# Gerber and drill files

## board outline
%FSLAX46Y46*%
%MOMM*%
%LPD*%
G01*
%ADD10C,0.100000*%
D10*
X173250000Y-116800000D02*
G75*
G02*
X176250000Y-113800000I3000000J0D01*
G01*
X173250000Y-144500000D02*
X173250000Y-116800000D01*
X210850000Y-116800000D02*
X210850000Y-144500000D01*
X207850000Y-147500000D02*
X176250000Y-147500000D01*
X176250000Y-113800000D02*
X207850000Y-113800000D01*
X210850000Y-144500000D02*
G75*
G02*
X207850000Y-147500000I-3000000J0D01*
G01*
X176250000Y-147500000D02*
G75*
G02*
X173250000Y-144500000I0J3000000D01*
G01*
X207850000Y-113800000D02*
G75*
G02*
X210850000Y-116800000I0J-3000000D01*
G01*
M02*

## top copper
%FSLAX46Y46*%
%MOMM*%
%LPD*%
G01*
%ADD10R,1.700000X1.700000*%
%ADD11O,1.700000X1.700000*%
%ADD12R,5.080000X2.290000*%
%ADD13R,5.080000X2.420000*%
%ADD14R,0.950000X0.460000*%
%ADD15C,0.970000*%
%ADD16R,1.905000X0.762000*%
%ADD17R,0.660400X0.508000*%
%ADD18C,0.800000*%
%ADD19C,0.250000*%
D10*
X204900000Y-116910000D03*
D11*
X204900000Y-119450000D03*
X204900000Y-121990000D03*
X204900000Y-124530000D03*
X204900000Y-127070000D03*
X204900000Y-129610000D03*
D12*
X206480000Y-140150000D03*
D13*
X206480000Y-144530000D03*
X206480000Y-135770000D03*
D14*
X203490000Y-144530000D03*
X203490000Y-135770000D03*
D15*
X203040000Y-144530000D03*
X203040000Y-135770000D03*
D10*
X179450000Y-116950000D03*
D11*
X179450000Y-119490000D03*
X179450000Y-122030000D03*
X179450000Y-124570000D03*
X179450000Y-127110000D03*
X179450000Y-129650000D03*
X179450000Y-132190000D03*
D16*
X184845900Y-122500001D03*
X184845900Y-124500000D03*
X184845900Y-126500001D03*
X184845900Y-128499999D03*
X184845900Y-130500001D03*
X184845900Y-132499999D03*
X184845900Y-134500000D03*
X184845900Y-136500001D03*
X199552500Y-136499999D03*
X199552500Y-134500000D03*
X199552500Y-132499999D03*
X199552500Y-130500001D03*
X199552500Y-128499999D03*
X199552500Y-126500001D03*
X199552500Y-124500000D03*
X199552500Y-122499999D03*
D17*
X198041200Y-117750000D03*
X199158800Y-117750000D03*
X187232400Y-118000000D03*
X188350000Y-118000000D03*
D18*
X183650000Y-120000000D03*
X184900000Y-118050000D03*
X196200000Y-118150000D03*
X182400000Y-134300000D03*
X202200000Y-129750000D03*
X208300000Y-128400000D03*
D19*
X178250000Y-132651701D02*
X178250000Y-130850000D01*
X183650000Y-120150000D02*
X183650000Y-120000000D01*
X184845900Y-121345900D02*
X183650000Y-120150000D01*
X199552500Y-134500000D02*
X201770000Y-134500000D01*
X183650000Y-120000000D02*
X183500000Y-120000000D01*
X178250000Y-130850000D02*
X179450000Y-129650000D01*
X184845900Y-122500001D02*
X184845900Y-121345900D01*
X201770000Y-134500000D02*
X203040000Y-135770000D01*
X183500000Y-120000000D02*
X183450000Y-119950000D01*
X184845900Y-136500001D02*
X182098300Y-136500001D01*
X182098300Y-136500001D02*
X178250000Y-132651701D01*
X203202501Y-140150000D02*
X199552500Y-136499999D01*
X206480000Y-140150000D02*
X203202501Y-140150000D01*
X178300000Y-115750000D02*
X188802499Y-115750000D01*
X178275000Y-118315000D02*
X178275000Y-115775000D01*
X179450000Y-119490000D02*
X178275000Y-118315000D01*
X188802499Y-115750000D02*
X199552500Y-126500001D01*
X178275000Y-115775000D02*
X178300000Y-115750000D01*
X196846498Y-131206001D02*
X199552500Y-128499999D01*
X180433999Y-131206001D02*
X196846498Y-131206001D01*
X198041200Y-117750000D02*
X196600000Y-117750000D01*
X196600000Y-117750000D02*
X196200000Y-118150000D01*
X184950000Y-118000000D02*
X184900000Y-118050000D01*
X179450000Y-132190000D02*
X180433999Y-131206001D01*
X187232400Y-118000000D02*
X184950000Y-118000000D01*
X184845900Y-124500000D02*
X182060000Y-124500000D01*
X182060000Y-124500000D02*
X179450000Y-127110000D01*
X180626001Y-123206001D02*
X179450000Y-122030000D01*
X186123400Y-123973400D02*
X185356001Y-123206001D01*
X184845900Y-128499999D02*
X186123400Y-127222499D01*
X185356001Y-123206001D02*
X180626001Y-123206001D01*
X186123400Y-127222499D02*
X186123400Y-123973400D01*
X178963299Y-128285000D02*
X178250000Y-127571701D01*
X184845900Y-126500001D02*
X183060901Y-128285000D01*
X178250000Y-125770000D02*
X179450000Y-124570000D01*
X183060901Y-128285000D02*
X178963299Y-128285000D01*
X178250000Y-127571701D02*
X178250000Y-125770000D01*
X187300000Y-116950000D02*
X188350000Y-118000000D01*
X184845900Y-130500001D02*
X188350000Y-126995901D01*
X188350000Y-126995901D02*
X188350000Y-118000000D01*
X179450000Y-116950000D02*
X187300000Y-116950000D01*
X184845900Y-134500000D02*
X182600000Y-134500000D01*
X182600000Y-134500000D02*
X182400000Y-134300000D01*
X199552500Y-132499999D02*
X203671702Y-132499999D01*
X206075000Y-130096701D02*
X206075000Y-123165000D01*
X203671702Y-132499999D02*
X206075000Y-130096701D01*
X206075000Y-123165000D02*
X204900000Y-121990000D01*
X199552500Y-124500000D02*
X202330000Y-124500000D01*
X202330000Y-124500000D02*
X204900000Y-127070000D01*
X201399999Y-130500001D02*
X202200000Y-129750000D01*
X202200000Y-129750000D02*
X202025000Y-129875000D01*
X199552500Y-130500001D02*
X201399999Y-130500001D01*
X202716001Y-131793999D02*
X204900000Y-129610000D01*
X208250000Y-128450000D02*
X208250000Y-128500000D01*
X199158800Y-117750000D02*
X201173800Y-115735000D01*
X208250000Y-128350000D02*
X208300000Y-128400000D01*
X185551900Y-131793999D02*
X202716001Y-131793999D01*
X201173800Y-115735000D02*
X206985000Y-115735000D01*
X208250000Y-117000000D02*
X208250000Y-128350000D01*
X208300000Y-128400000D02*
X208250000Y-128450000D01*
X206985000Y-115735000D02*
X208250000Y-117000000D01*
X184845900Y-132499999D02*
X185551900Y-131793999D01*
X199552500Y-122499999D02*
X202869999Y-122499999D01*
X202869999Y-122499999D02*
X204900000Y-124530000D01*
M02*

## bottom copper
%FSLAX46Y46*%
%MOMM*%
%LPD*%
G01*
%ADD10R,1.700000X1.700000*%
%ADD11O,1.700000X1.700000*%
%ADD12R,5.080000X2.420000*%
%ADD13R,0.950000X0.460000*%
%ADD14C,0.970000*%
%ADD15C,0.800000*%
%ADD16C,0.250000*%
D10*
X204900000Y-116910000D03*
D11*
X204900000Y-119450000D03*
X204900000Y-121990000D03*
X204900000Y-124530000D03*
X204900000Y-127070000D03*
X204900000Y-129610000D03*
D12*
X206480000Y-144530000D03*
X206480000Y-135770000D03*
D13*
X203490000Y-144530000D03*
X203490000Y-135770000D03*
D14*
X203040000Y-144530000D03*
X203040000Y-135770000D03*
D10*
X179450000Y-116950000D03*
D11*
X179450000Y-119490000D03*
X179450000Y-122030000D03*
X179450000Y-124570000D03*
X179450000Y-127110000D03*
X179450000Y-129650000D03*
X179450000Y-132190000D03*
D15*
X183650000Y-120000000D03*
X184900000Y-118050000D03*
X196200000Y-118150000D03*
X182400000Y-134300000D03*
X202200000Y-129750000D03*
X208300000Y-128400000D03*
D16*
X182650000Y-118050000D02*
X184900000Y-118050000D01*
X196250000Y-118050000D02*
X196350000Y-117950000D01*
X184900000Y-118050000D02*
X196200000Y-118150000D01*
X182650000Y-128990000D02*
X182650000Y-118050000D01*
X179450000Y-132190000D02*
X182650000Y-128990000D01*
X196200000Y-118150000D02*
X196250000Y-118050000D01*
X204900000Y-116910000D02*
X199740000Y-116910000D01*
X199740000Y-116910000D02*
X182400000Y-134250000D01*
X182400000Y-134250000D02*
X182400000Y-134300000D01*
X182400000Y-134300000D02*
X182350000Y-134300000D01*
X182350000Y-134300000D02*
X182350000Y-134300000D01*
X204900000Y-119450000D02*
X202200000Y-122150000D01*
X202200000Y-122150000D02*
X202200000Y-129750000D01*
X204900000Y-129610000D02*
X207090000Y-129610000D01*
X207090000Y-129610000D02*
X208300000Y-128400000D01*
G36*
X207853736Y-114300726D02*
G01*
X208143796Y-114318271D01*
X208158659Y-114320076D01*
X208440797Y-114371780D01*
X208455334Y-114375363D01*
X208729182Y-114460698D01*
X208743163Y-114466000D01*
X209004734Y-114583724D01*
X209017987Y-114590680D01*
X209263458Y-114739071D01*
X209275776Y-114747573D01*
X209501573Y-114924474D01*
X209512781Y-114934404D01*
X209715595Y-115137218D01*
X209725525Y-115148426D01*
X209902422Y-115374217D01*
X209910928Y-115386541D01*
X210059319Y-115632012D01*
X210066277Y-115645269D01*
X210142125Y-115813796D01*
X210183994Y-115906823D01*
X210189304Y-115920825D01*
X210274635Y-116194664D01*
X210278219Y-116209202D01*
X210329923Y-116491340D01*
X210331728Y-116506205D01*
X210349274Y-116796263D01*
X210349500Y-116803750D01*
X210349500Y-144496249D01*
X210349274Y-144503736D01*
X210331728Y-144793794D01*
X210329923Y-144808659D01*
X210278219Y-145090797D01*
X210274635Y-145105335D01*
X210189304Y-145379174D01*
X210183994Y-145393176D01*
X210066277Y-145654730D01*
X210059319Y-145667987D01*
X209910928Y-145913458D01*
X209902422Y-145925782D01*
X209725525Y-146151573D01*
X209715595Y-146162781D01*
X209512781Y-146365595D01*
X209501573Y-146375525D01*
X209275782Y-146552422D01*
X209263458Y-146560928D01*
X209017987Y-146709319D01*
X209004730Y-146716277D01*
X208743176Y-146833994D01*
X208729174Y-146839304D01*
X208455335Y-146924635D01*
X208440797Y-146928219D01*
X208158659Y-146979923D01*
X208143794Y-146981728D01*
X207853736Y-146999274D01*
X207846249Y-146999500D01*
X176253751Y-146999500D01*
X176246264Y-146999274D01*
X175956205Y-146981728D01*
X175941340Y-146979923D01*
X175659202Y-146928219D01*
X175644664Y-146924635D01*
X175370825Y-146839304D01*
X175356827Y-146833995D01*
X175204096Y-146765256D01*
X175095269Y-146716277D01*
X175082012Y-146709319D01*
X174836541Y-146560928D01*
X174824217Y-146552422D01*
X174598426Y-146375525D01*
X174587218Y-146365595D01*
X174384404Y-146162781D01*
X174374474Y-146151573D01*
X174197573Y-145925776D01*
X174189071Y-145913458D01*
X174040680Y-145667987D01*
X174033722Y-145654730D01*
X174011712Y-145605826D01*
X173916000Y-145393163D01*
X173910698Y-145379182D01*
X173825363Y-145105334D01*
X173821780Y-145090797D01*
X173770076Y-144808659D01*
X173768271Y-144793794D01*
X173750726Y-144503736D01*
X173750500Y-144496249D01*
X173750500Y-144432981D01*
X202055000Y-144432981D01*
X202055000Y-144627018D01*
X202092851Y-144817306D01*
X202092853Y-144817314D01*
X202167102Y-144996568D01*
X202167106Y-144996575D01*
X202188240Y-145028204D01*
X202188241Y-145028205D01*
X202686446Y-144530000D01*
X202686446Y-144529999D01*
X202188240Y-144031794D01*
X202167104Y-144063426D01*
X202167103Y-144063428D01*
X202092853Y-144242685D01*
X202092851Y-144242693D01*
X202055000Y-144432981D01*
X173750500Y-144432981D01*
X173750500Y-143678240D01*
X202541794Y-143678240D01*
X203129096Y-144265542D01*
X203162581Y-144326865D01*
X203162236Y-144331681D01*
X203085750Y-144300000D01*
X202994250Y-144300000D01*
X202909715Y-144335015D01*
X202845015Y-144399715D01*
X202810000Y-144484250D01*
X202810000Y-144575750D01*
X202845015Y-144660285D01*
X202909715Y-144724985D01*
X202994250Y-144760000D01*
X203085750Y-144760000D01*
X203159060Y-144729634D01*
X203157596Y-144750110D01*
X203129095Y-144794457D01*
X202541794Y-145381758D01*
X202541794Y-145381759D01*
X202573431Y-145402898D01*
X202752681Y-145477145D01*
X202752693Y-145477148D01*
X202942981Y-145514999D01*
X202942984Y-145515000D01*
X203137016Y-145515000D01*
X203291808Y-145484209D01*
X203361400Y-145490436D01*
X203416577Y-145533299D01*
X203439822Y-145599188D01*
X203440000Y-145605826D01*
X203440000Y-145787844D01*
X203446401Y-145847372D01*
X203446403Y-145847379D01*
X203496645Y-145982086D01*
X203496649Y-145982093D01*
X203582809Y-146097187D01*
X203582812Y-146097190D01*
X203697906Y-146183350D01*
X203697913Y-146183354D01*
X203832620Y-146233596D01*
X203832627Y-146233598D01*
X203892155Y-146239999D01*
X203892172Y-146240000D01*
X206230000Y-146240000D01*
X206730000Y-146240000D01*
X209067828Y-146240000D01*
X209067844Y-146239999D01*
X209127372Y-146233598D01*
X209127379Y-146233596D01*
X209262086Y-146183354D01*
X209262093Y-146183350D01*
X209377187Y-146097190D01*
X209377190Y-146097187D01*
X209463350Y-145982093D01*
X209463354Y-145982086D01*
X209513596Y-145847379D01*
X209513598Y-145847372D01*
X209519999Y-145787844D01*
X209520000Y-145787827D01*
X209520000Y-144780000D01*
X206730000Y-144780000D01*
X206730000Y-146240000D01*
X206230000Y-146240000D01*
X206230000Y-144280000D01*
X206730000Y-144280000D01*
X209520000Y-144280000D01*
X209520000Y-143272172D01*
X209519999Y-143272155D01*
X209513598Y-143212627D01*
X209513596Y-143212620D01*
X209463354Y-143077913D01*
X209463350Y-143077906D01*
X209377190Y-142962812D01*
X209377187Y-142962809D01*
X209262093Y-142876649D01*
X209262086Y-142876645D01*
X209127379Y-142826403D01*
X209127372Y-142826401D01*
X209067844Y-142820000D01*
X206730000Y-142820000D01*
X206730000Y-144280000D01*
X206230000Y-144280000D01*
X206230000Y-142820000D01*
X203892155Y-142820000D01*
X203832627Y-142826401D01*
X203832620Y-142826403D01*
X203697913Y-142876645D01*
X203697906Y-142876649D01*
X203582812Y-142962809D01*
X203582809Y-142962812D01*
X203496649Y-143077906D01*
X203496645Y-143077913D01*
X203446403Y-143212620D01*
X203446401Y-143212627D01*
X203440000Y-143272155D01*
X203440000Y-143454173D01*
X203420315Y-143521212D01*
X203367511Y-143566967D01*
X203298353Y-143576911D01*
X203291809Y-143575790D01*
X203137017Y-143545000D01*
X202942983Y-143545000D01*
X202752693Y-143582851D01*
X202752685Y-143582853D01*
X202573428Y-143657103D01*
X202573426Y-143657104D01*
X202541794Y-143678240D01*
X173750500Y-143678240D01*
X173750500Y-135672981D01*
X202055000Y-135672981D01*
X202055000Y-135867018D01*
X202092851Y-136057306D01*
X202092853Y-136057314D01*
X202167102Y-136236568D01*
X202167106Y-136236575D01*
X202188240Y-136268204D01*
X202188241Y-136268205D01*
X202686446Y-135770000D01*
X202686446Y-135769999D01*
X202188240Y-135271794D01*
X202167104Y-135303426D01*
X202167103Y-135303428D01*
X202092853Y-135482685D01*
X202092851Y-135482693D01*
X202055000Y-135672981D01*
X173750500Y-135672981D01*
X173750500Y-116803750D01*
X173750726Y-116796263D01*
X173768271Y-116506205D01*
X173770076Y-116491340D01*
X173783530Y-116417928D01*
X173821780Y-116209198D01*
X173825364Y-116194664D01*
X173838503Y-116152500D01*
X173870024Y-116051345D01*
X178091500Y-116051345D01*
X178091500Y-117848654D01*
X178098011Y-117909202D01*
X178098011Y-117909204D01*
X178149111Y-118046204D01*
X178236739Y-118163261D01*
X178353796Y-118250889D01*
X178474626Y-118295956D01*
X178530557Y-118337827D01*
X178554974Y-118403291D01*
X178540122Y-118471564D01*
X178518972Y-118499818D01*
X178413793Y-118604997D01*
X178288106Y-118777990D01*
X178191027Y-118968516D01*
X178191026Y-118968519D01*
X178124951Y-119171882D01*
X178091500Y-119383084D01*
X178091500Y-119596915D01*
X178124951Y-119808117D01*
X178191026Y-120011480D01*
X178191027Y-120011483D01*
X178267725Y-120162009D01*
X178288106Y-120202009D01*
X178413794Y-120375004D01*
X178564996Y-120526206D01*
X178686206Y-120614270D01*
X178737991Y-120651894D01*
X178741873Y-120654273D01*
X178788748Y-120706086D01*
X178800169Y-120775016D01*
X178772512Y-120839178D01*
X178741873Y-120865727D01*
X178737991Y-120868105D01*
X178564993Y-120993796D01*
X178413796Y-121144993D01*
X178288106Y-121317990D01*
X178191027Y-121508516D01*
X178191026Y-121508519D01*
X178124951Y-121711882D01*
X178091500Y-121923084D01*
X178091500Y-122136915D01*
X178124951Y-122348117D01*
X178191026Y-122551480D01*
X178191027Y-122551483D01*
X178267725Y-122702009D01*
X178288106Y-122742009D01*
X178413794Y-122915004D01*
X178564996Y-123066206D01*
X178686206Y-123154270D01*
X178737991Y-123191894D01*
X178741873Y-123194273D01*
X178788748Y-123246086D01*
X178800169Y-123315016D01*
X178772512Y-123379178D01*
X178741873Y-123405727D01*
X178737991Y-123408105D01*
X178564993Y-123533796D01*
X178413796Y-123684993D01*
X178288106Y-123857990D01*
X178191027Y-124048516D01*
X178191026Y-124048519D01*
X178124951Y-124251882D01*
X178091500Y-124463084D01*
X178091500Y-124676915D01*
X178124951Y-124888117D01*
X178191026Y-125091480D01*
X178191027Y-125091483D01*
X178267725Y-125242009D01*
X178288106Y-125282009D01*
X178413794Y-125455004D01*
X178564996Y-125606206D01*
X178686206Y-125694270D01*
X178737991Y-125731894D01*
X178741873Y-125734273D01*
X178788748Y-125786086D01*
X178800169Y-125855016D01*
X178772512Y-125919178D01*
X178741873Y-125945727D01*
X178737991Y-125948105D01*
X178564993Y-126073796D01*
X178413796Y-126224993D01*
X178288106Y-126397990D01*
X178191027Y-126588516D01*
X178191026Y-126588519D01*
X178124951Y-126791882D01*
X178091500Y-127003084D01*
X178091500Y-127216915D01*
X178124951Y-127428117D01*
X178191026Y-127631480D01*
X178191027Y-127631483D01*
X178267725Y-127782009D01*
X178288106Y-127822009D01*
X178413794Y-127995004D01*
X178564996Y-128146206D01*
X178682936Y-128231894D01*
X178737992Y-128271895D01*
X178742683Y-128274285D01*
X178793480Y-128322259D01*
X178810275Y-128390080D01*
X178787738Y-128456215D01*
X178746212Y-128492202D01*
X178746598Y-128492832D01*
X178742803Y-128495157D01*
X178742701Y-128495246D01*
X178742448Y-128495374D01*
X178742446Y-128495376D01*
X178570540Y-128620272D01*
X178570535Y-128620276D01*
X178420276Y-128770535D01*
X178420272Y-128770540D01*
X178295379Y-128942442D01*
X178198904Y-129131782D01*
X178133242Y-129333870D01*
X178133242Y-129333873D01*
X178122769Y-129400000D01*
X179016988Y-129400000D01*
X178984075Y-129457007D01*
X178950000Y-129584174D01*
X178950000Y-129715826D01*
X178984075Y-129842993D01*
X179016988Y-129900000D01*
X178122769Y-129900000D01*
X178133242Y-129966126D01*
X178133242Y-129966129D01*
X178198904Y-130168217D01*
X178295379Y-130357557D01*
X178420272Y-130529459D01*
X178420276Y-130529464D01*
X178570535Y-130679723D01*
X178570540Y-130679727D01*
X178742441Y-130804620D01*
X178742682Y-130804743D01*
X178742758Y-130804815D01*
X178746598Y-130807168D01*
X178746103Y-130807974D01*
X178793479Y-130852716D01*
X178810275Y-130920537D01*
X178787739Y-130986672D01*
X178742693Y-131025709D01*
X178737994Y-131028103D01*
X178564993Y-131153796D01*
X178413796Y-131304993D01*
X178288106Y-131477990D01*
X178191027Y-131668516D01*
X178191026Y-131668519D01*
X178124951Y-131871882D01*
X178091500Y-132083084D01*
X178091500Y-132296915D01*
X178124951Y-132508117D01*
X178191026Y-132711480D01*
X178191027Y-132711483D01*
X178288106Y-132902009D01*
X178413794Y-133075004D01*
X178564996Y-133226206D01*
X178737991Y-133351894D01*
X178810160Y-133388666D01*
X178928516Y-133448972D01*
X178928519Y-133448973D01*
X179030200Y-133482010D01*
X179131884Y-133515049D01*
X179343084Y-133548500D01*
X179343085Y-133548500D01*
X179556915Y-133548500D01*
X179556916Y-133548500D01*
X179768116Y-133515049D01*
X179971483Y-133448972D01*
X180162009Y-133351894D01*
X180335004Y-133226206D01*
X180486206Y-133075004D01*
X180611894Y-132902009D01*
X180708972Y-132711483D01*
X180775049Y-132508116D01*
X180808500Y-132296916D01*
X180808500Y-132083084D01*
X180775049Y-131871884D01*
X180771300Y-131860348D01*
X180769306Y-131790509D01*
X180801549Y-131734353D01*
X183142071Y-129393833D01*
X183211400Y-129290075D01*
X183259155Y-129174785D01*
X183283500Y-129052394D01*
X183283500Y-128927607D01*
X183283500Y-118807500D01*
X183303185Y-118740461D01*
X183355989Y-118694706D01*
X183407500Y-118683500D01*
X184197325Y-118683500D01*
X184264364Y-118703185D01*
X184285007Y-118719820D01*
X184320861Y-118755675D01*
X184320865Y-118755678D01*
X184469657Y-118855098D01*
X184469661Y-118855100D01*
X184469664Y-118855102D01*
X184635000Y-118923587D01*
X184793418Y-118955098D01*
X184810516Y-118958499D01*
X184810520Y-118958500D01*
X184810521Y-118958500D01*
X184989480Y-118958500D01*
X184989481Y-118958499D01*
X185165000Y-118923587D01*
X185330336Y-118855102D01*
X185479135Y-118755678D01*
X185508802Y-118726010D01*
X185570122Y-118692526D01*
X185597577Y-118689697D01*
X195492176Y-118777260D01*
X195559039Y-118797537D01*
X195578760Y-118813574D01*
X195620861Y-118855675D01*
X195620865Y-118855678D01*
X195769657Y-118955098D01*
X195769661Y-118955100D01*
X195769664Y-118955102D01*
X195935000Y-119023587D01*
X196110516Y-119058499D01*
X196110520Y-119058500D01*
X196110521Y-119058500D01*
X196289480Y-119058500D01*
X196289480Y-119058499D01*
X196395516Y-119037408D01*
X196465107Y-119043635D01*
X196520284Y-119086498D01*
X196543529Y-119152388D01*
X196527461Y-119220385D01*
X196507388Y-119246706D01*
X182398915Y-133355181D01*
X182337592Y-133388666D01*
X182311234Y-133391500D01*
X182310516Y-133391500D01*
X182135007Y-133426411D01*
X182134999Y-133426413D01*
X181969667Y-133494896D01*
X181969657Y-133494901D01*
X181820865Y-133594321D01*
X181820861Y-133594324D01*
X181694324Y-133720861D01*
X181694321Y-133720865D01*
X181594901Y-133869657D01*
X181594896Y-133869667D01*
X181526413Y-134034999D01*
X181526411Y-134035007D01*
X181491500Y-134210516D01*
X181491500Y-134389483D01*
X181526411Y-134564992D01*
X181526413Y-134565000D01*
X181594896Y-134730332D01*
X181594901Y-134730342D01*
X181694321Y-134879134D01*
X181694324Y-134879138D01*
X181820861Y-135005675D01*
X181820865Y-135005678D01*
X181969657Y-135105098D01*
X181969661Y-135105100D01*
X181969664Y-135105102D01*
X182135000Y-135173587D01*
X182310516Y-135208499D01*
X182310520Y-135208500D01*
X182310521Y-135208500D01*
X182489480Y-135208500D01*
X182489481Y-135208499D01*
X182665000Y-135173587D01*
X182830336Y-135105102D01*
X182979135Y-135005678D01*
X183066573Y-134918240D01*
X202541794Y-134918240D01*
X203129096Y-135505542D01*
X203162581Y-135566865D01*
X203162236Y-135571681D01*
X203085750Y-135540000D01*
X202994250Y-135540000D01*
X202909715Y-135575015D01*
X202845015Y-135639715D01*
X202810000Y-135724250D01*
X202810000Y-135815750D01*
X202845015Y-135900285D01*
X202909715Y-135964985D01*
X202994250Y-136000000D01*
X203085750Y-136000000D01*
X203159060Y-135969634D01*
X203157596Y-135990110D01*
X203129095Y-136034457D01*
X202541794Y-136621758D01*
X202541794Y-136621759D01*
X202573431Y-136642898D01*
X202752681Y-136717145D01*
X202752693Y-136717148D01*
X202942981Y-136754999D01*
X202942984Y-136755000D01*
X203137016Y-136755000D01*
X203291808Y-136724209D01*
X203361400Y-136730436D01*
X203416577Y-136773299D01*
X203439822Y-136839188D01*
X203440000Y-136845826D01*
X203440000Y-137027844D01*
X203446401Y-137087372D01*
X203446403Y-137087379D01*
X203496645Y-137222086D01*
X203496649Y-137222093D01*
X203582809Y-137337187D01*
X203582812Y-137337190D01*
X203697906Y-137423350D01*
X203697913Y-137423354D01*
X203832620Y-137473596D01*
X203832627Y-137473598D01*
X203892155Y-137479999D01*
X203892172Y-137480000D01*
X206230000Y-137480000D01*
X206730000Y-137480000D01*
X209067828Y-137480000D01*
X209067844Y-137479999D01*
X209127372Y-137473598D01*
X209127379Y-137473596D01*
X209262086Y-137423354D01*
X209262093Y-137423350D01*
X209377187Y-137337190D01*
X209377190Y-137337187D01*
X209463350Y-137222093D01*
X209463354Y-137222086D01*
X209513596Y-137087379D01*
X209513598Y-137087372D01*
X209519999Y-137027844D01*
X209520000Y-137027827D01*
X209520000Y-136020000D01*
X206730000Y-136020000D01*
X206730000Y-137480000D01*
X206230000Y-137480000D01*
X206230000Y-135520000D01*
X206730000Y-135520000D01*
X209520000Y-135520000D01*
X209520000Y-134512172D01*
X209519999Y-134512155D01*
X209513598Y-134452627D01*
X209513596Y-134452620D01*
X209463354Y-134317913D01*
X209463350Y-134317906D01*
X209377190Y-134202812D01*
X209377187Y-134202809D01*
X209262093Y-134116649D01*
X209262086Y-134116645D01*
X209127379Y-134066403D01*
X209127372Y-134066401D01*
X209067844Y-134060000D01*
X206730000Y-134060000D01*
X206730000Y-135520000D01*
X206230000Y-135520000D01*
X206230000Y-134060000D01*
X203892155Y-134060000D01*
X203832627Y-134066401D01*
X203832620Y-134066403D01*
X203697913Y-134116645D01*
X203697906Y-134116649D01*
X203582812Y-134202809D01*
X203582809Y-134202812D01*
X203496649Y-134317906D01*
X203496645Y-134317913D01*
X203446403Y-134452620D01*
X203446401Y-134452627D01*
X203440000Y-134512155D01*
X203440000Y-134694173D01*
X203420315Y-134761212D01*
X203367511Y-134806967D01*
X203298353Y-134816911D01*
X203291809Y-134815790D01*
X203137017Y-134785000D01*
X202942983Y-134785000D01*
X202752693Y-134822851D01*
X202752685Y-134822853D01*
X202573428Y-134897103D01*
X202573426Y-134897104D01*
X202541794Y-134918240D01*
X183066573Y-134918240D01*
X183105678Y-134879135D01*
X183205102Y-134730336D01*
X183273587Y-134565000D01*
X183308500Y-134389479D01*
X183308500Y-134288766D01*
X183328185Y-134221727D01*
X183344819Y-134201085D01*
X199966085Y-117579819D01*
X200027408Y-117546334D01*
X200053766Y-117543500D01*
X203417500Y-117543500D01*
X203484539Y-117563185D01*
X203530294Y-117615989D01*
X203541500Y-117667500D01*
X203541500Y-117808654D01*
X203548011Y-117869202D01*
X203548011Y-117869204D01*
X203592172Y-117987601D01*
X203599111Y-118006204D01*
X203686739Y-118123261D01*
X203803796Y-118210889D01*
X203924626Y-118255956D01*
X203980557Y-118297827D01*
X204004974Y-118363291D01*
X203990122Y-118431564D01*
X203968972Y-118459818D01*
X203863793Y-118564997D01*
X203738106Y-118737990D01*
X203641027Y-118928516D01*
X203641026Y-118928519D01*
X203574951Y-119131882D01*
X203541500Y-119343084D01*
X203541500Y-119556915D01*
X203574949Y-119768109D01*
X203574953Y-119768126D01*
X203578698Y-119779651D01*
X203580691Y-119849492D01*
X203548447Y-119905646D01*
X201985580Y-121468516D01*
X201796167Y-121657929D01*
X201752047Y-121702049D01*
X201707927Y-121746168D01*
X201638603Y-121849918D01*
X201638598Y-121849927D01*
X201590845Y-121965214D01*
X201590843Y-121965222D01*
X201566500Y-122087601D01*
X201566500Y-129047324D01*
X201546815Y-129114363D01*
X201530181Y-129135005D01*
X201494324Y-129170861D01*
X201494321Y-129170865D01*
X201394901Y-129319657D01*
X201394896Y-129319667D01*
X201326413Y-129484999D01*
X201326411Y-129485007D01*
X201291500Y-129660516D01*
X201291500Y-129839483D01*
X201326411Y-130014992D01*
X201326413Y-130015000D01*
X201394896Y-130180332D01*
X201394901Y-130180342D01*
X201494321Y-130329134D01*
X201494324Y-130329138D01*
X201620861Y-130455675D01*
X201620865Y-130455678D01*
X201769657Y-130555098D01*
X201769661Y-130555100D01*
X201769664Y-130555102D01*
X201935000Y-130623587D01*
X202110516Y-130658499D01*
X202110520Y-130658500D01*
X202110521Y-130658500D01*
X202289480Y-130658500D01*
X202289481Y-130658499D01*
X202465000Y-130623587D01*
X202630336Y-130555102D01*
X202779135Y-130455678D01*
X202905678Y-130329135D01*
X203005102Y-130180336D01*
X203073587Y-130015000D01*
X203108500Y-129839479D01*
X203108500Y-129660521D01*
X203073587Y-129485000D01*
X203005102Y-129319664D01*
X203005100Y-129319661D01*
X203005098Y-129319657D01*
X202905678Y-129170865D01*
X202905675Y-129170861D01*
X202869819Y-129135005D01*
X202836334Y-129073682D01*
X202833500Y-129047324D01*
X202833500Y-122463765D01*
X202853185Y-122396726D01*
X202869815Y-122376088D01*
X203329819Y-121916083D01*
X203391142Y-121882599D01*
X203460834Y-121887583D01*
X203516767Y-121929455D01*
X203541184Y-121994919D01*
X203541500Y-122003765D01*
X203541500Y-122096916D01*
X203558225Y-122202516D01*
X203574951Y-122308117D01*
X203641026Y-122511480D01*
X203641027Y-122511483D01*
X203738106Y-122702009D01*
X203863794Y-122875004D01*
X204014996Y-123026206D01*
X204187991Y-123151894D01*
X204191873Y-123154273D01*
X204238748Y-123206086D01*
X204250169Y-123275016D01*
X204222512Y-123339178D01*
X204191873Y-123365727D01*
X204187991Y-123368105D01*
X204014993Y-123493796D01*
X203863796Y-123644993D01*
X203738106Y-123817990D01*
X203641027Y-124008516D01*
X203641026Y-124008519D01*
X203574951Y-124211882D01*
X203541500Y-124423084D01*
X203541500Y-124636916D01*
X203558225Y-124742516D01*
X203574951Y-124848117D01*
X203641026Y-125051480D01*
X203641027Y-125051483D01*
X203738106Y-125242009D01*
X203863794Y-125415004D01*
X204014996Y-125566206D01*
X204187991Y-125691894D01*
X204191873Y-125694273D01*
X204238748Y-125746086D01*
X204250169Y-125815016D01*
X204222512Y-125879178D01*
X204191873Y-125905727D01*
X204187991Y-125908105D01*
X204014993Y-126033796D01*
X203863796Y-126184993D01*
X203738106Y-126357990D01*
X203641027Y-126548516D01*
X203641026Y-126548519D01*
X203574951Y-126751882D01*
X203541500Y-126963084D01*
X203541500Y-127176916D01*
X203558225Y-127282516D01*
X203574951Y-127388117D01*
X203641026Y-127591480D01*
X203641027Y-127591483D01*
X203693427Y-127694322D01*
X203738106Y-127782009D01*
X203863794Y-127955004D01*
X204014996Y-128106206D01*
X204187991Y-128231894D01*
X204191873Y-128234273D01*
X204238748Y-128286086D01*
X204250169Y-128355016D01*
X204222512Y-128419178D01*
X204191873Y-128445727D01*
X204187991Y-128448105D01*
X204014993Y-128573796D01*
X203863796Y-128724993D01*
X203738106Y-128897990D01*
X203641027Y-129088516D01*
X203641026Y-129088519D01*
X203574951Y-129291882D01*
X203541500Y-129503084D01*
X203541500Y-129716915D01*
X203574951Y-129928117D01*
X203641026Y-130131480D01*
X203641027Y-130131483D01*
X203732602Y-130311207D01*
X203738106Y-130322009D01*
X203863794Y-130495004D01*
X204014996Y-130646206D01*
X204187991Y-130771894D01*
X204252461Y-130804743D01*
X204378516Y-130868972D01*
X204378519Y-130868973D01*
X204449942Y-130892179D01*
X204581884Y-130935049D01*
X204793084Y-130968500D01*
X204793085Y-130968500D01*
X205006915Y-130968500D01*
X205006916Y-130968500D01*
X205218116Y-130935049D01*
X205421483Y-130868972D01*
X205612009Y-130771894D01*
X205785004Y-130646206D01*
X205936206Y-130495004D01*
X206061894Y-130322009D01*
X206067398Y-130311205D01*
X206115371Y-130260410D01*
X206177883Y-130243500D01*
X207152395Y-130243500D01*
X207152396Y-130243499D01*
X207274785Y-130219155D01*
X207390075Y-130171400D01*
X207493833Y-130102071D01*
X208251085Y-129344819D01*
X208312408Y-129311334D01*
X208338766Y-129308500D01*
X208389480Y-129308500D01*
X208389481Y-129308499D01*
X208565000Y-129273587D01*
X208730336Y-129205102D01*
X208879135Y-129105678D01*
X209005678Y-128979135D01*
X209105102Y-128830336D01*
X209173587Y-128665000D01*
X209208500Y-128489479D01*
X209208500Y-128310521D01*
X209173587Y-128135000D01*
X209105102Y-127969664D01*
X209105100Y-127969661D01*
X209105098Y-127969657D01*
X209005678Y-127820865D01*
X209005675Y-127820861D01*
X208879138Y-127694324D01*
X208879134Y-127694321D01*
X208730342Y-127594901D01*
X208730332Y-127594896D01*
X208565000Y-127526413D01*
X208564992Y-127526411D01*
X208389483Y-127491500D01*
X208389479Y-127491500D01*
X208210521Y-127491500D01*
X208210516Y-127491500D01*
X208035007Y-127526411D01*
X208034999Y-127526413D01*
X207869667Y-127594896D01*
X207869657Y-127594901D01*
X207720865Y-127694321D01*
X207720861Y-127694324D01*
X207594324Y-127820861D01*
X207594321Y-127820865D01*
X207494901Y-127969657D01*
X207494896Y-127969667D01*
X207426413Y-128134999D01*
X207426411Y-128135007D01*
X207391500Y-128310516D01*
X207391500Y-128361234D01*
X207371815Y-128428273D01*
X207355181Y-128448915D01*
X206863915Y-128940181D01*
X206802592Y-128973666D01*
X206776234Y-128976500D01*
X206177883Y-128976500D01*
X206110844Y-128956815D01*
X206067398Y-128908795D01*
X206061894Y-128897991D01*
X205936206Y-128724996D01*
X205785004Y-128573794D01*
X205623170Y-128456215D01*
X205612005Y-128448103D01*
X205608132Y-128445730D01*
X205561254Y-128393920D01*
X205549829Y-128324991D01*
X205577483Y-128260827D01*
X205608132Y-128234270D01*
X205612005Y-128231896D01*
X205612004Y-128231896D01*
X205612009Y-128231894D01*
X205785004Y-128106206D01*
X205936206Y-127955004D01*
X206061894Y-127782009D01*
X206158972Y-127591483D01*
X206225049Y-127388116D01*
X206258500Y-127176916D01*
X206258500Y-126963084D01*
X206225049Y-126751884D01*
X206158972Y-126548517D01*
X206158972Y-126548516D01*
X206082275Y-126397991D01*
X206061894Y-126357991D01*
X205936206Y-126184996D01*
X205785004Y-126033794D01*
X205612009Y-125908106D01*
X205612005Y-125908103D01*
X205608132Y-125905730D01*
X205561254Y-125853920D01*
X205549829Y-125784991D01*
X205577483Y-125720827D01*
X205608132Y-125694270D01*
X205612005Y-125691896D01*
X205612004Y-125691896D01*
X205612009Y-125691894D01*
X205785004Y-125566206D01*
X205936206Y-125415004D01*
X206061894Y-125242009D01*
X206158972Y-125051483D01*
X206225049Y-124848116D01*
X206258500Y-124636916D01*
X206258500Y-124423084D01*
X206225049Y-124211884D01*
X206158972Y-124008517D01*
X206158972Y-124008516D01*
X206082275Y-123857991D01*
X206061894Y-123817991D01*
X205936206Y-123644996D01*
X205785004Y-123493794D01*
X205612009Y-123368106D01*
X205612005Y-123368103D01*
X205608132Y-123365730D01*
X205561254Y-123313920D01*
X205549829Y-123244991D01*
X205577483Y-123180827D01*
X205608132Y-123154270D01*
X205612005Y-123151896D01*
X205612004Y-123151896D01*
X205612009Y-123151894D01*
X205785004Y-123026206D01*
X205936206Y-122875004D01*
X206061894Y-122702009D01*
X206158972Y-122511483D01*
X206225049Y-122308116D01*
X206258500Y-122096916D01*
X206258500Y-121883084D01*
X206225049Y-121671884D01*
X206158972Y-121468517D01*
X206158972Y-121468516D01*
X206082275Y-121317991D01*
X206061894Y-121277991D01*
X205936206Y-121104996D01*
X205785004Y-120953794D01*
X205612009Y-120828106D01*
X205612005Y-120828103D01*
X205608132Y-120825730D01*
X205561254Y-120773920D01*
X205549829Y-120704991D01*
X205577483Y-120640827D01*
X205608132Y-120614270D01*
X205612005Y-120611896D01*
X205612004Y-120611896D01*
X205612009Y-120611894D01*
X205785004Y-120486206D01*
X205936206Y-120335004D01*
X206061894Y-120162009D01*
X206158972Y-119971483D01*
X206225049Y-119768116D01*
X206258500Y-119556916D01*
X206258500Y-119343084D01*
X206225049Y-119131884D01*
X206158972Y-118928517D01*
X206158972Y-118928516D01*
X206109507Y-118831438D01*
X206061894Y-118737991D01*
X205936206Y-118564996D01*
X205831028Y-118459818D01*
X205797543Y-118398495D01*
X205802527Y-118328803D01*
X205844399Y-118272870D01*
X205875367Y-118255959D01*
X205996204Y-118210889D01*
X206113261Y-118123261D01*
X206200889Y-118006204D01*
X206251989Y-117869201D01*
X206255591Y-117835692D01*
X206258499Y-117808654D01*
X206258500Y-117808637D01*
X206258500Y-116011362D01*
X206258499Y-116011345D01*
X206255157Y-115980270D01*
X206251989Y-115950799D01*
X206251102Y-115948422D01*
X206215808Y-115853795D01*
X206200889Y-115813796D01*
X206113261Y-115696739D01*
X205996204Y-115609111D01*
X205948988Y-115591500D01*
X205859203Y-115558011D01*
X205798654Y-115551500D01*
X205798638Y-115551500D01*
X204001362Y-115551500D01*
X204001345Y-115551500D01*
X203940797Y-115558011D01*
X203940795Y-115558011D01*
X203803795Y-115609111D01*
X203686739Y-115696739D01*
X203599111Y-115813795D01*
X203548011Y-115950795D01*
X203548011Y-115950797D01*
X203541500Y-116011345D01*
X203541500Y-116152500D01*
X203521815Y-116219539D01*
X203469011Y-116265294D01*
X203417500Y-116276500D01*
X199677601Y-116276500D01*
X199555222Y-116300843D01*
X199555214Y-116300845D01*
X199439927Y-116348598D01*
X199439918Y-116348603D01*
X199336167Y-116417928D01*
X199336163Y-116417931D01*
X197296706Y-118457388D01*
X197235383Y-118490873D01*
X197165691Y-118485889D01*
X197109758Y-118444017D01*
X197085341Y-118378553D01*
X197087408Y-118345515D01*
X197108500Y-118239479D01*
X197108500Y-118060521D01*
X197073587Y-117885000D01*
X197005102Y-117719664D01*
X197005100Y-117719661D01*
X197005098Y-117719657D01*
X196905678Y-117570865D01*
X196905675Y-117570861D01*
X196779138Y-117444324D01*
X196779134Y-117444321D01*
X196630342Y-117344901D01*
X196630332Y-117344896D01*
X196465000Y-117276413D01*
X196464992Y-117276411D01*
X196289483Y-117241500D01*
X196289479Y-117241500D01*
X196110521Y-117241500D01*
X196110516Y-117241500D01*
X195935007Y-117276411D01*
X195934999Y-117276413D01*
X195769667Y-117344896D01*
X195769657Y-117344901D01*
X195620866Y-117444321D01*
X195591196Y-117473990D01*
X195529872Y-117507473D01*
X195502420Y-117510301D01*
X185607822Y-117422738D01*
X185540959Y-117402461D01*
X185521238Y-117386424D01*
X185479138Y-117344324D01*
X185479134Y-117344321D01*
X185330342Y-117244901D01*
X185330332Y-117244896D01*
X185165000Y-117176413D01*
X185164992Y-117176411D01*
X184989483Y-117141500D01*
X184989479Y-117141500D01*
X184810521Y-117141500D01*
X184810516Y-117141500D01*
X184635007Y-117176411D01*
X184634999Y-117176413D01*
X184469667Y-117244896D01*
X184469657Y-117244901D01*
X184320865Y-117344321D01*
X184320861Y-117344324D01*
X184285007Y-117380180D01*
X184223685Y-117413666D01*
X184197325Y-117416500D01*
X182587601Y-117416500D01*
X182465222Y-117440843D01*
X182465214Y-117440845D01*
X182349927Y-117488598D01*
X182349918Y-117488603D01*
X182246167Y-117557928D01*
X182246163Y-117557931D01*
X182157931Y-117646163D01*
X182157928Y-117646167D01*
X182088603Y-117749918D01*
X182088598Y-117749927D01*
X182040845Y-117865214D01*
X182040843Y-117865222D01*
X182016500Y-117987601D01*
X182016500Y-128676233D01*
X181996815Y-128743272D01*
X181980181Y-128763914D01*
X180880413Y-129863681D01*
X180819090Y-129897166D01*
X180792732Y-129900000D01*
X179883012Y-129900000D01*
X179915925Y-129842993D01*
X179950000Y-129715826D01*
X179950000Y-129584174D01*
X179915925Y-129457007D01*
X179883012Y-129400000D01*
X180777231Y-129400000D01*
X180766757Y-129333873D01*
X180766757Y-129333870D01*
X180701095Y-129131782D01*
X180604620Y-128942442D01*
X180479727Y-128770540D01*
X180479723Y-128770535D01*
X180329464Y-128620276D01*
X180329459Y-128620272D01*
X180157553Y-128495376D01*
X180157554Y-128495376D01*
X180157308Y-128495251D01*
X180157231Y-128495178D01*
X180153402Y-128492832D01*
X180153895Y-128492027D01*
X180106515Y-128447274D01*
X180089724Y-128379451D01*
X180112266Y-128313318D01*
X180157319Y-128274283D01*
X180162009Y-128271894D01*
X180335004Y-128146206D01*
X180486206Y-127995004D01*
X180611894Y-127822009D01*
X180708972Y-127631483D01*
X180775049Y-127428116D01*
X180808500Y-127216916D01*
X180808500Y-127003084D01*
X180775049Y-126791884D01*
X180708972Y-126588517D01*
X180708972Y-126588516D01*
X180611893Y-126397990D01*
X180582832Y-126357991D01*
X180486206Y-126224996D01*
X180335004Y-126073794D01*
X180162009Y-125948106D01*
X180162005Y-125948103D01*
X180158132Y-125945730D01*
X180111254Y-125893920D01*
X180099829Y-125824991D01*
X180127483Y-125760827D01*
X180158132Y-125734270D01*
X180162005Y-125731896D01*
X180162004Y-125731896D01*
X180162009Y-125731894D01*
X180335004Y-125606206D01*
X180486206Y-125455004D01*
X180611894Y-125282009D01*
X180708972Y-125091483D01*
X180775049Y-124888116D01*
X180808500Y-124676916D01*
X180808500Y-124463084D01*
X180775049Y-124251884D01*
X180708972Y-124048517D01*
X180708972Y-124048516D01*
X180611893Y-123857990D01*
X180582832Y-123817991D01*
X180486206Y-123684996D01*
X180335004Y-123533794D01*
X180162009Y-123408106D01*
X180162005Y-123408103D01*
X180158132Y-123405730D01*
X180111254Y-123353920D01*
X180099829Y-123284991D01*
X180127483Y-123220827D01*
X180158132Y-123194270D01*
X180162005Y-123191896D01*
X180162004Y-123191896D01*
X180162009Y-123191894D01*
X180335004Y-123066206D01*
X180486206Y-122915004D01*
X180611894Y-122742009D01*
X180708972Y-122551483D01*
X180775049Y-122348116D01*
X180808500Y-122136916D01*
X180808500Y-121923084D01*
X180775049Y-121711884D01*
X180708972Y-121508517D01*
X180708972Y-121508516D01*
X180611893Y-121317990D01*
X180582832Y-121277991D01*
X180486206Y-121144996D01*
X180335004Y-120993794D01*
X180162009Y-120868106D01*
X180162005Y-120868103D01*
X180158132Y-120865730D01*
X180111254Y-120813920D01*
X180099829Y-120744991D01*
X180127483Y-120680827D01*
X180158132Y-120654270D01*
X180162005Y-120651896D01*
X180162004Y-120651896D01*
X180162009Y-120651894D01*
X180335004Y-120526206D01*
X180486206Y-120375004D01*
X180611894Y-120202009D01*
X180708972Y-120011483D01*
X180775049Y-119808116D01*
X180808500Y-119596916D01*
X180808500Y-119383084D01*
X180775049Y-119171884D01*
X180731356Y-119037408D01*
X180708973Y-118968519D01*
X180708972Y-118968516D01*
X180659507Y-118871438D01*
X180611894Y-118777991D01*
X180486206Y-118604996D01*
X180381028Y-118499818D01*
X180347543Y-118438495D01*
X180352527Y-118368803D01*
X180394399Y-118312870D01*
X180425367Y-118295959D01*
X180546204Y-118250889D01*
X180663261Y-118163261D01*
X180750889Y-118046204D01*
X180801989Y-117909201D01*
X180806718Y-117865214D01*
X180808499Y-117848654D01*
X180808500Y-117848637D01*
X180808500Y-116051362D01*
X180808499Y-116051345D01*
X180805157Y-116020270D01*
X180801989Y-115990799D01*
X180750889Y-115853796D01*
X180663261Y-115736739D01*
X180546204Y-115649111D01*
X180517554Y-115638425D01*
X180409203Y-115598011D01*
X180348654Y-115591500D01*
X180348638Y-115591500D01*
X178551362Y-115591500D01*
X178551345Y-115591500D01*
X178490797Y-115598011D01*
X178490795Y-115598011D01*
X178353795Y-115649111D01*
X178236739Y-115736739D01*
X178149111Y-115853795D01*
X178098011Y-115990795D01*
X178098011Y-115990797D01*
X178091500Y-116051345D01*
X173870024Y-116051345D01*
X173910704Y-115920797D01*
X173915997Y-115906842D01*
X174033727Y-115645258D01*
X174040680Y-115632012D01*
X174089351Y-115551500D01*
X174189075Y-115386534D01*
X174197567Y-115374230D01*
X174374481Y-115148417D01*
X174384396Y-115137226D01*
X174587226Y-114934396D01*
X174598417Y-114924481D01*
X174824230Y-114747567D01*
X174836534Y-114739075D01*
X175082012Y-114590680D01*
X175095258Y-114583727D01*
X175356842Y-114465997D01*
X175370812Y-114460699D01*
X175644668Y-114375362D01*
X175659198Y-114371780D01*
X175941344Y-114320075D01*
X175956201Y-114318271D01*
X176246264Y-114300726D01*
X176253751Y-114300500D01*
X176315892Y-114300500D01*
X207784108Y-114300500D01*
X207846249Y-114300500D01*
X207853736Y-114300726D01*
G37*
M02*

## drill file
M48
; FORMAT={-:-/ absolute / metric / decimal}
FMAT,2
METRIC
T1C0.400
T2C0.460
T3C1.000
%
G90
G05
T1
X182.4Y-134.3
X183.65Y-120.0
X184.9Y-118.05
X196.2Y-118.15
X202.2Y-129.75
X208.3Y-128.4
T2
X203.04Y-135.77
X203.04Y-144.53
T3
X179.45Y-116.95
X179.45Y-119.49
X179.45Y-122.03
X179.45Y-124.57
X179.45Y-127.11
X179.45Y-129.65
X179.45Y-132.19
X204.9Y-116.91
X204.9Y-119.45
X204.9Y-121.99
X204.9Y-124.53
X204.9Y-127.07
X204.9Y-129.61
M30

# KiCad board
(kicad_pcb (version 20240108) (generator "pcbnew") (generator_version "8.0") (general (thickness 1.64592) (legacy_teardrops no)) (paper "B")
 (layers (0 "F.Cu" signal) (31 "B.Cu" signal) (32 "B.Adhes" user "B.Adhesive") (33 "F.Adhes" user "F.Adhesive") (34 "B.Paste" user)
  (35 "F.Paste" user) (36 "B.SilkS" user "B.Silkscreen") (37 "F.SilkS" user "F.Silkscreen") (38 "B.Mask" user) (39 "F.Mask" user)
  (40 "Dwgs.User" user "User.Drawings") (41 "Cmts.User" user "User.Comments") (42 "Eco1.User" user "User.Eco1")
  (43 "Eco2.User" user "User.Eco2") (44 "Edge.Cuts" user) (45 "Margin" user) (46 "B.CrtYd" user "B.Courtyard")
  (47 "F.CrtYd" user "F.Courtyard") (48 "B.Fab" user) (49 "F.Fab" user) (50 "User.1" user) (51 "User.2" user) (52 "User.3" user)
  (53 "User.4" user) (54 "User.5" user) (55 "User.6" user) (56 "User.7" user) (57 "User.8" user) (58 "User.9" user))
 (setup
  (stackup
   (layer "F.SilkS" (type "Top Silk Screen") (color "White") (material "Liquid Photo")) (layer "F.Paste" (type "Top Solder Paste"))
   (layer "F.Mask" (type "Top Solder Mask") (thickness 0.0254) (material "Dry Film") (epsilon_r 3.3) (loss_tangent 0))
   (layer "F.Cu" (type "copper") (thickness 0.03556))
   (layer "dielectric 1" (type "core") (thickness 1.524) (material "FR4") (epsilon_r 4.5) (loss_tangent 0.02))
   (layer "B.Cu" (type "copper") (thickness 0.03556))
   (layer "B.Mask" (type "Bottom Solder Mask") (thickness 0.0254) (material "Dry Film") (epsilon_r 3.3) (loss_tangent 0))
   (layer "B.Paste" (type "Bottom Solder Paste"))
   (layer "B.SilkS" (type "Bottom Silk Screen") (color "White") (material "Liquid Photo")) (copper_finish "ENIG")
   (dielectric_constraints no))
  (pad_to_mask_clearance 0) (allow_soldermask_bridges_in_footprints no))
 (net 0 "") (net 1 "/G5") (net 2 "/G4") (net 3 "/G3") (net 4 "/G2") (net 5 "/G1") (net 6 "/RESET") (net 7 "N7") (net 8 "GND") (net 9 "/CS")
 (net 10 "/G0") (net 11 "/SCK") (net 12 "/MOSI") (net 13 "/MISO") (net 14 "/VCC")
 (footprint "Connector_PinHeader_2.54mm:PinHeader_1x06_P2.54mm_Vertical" (layer "F.Cu") (at 204.9 116.91)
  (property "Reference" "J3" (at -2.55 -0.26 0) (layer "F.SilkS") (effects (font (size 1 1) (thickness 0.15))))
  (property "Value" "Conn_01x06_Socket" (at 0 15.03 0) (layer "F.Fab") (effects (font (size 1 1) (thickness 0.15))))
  (pad "1" thru_hole rect (at 0 0) (size 1.7 1.7) (drill 1) (layers "*.Cu" "*.Mask") (remove_unused_layers no) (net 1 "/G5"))
  (pad "2" thru_hole oval (at 0 2.54) (size 1.7 1.7) (drill 1) (layers "*.Cu" "*.Mask") (remove_unused_layers no) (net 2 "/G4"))
  (pad "3" thru_hole oval (at 0 5.08) (size 1.7 1.7) (drill 1) (layers "*.Cu" "*.Mask") (remove_unused_layers no) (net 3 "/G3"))
  (pad "4" thru_hole oval (at 0 7.62) (size 1.7 1.7) (drill 1) (layers "*.Cu" "*.Mask") (remove_unused_layers no) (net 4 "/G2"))
  (pad "5" thru_hole oval (at 0 10.16) (size 1.7 1.7) (drill 1) (layers "*.Cu" "*.Mask") (remove_unused_layers no) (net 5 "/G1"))
  (pad "6" thru_hole oval (at 0 12.7) (size 1.7 1.7) (drill 1) (layers "*.Cu" "*.Mask") (remove_unused_layers no) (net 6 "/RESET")))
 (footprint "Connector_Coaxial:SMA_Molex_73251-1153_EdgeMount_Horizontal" (layer "F.Cu") (at 204.76 140.15 180)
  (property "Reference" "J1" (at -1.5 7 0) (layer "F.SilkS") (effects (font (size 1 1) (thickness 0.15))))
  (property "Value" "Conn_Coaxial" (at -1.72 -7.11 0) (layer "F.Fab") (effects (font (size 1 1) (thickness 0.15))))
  (pad "1" smd rect (at -1.72 0 180) (size 5.08 2.29) (layers "F.Cu" "F.Paste" "F.Mask") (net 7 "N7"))
  (pad "2" smd rect (at -1.72 -4.38 180) (size 5.08 2.42) (layers "F.Cu" "F.Paste" "F.Mask") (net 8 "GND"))
  (pad "2" smd rect (at -1.72 -4.38 180) (size 5.08 2.42) (layers "B.Cu" "B.Paste" "B.Mask") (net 8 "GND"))
  (pad "2" smd rect (at -1.72 4.38 180) (size 5.08 2.42) (layers "F.Cu" "F.Paste" "F.Mask") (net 8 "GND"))
  (pad "2" smd rect (at -1.72 4.38 180) (size 5.08 2.42) (layers "B.Cu" "B.Paste" "B.Mask") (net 8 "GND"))
  (pad "2" smd rect (at 1.27 -4.38 180) (size 0.95 0.46) (layers "F.Cu") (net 8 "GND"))
  (pad "2" smd rect (at 1.27 -4.38 180) (size 0.95 0.46) (layers "B.Cu") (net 8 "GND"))
  (pad "2" smd rect (at 1.27 4.38 180) (size 0.95 0.46) (layers "F.Cu") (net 8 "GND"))
  (pad "2" smd rect (at 1.27 4.38 180) (size 0.95 0.46) (layers "B.Cu") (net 8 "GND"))
  (pad "2" thru_hole circle (at 1.72 -4.38 180) (size 0.97 0.97) (drill 0.46) (layers "*.Cu") (remove_unused_layers no) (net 8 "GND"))
  (pad "2" thru_hole circle (at 1.72 4.38 180) (size 0.97 0.97) (drill 0.46) (layers "*.Cu") (remove_unused_layers no) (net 8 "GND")))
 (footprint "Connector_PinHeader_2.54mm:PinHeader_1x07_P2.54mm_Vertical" (layer "F.Cu") (at 179.45 116.95)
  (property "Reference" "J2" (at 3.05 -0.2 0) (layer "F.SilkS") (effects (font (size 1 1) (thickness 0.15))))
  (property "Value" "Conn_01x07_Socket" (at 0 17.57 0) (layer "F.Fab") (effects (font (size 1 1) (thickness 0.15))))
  (pad "1" thru_hole rect (at 0 0) (size 1.7 1.7) (drill 1) (layers "*.Cu" "*.Mask") (remove_unused_layers no) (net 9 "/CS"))
  (pad "2" thru_hole oval (at 0 2.54) (size 1.7 1.7) (drill 1) (layers "*.Cu" "*.Mask") (remove_unused_layers no) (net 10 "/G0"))
  (pad "3" thru_hole oval (at 0 5.08) (size 1.7 1.7) (drill 1) (layers "*.Cu" "*.Mask") (remove_unused_layers no) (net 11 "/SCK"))
  (pad "4" thru_hole oval (at 0 7.62) (size 1.7 1.7) (drill 1) (layers "*.Cu" "*.Mask") (remove_unused_layers no) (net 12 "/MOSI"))
  (pad "5" thru_hole oval (at 0 10.16) (size 1.7 1.7) (drill 1) (layers "*.Cu" "*.Mask") (remove_unused_layers no) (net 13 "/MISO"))
  (pad "6" thru_hole oval (at 0 12.7) (size 1.7 1.7) (drill 1) (layers "*.Cu" "*.Mask") (remove_unused_layers no) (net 8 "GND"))
  (pad "7" thru_hole oval (at 0 15.24) (size 1.7 1.7) (drill 1) (layers "*.Cu" "*.Mask") (remove_unused_layers no) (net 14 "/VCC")))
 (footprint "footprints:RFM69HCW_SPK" (layer "F.Cu") (at 192.1992 129.5)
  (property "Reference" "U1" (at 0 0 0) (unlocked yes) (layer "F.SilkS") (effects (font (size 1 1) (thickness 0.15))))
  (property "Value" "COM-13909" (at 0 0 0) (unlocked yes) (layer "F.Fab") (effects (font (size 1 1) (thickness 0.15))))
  (pad "1" smd rect (at -7.3533 -6.999999) (size 1.905 0.762) (layers "F.Cu" "F.Paste" "F.Mask") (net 8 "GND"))
  (pad "2" smd rect (at -7.3533 -5) (size 1.905 0.762) (layers "F.Cu" "F.Paste" "F.Mask") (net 13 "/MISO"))
  (pad "3" smd rect (at -7.3533 -2.999999) (size 1.905 0.762) (layers "F.Cu" "F.Paste" "F.Mask") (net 12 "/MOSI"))
  (pad "4" smd rect (at -7.3533 -1.000001) (size 1.905 0.762) (layers "F.Cu" "F.Paste" "F.Mask") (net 11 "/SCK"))
  (pad "5" smd rect (at -7.3533 1.000001) (size 1.905 0.762) (layers "F.Cu" "F.Paste" "F.Mask") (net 9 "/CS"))
  (pad "6" smd rect (at -7.3533 2.999999) (size 1.905 0.762) (layers "F.Cu" "F.Paste" "F.Mask") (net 6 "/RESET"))
  (pad "7" smd rect (at -7.3533 5) (size 1.905 0.762) (layers "F.Cu" "F.Paste" "F.Mask") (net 1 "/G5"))
  (pad "8" smd rect (at -7.3533 7.000001) (size 1.905 0.762) (layers "F.Cu" "F.Paste" "F.Mask") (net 8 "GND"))
  (pad "9" smd rect (at 7.3533 6.999999) (size 1.905 0.762) (layers "F.Cu" "F.Paste" "F.Mask") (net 7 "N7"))
  (pad "10" smd rect (at 7.3533 5) (size 1.905 0.762) (layers "F.Cu" "F.Paste" "F.Mask") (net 8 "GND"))
  (pad "11" smd rect (at 7.3533 2.999999) (size 1.905 0.762) (layers "F.Cu" "F.Paste" "F.Mask") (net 3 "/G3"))
  (pad "12" smd rect (at 7.3533 1.000001) (size 1.905 0.762) (layers "F.Cu" "F.Paste" "F.Mask") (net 2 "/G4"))
  (pad "13" smd rect (at 7.3533 -1.000001) (size 1.905 0.762) (layers "F.Cu" "F.Paste" "F.Mask") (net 14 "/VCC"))
  (pad "14" smd rect (at 7.3533 -2.999999) (size 1.905 0.762) (layers "F.Cu" "F.Paste" "F.Mask") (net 10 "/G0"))
  (pad "15" smd rect (at 7.3533 -5) (size 1.905 0.762) (layers "F.Cu" "F.Paste" "F.Mask") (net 5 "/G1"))
  (pad "16" smd rect (at 7.3533 -7.000001) (size 1.905 0.762) (layers "F.Cu" "F.Paste" "F.Mask") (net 4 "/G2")))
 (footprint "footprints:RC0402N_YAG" (layer "F.Cu") (at 198.6 117.75)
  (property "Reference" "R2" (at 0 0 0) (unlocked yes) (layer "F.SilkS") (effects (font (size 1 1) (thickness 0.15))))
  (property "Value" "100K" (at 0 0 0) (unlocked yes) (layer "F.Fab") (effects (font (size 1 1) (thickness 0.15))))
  (pad "1" smd rect (at -0.5588 0) (size 0.6604 0.508) (layers "F.Cu" "F.Paste" "F.Mask") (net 14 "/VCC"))
  (pad "2" smd rect (at 0.5588 0) (size 0.6604 0.508) (layers "F.Cu" "F.Paste" "F.Mask") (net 6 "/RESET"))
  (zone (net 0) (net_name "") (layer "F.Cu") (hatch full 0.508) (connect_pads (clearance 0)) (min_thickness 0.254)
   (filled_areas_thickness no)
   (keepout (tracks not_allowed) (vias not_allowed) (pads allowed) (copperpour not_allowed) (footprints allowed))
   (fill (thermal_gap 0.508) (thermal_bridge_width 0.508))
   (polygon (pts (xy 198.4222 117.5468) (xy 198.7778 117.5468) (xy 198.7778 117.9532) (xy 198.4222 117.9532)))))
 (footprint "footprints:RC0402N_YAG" (layer "F.Cu") (at 187.7912 118)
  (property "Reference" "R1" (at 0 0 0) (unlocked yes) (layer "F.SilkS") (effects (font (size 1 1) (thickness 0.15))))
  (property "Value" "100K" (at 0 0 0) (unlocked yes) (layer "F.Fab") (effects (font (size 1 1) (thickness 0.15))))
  (pad "1" smd rect (at -0.5588 0) (size 0.6604 0.508) (layers "F.Cu" "F.Paste" "F.Mask") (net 14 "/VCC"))
  (pad "2" smd rect (at 0.5588 0) (size 0.6604 0.508) (layers "F.Cu" "F.Paste" "F.Mask") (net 9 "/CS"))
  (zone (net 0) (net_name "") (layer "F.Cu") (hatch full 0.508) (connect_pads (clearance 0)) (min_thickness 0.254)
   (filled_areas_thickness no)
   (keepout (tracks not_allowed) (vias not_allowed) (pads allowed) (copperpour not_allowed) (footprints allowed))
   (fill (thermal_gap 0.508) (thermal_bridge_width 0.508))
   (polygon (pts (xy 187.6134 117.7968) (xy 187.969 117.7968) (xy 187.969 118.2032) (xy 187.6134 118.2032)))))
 (gr_arc (start 173.25 116.8) (mid 174.12868 114.67868) (end 176.25 113.8) (stroke (width 0.1) (type default)) (layer "Edge.Cuts"))
 (gr_line (start 173.25 144.5) (end 173.25 116.8) (stroke (width 0.1) (type default)) (layer "Edge.Cuts"))
 (gr_line (start 210.85 116.8) (end 210.85 144.5) (stroke (width 0.1) (type default)) (layer "Edge.Cuts"))
 (gr_line (start 207.85 147.5) (end 176.25 147.5) (stroke (width 0.1) (type default)) (layer "Edge.Cuts"))
 (gr_line (start 176.25 113.8) (end 207.85 113.8) (stroke (width 0.1) (type default)) (layer "Edge.Cuts"))
 (gr_arc (start 210.85 144.5) (mid 209.97132 146.62132) (end 207.85 147.5) (stroke (width 0.1) (type default)) (layer "Edge.Cuts"))
 (gr_arc (start 176.25 147.5) (mid 174.12868 146.62132) (end 173.25 144.5) (stroke (width 0.1) (type default)) (layer "Edge.Cuts"))
 (gr_arc (start 207.85 113.8) (mid 209.97132 114.67868) (end 210.85 116.8) (stroke (width 0.1) (type default)) (layer "Edge.Cuts"))
 (segment (start 178.25 132.651701) (end 178.25 130.85) (width 0.25) (layer "F.Cu") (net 8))
 (segment (start 183.65 120.15) (end 183.65 120) (width 0.25) (layer "F.Cu") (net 8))
 (segment (start 184.8459 121.3459) (end 183.65 120.15) (width 0.25) (layer "F.Cu") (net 8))
 (segment (start 199.5525 134.5) (end 201.77 134.5) (width 0.25) (layer "F.Cu") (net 8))
 (segment (start 183.65 120) (end 183.5 120) (width 0.25) (layer "F.Cu") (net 8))
 (segment (start 178.25 130.85) (end 179.45 129.65) (width 0.25) (layer "F.Cu") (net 8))
 (segment (start 184.8459 122.500001) (end 184.8459 121.3459) (width 0.25) (layer "F.Cu") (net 8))
 (segment (start 201.77 134.5) (end 203.04 135.77) (width 0.25) (layer "F.Cu") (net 8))
 (segment (start 183.5 120) (end 183.45 119.95) (width 0.25) (layer "F.Cu") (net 8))
 (segment (start 184.8459 136.500001) (end 182.0983 136.500001) (width 0.25) (layer "F.Cu") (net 8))
 (segment (start 182.0983 136.500001) (end 178.25 132.651701) (width 0.25) (layer "F.Cu") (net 8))
 (via (at 183.65 120) (size 0.8) (drill 0.4) (layers "F.Cu" "B.Cu") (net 8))
 (segment (start 203.202501 140.15) (end 199.5525 136.499999) (width 0.25) (layer "F.Cu") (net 7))
 (segment (start 206.48 140.15) (end 203.202501 140.15) (width 0.25) (layer "F.Cu") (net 7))
 (segment (start 178.3 115.75) (end 188.802499 115.75) (width 0.25) (layer "F.Cu") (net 10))
 (segment (start 178.275 118.315) (end 178.275 115.775) (width 0.25) (layer "F.Cu") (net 10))
 (segment (start 179.45 119.49) (end 178.275 118.315) (width 0.25) (layer "F.Cu") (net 10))
 (segment (start 188.802499 115.75) (end 199.5525 126.500001) (width 0.25) (layer "F.Cu") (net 10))
 (segment (start 178.275 115.775) (end 178.3 115.75) (width 0.25) (layer "F.Cu") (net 10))
 (segment (start 196.846498 131.206001) (end 199.5525 128.499999) (width 0.25) (layer "F.Cu") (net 14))
 (segment (start 180.433999 131.206001) (end 196.846498 131.206001) (width 0.25) (layer "F.Cu") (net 14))
 (segment (start 198.0412 117.75) (end 196.6 117.75) (width 0.25) (layer "F.Cu") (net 14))
 (segment (start 196.6 117.75) (end 196.2 118.15) (width 0.25) (layer "F.Cu") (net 14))
 (segment (start 184.95 118) (end 184.9 118.05) (width 0.25) (layer "F.Cu") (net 14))
 (segment (start 179.45 132.19) (end 180.433999 131.206001) (width 0.25) (layer "F.Cu") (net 14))
 (segment (start 187.2324 118) (end 184.95 118) (width 0.25) (layer "F.Cu") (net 14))
 (via (at 184.9 118.05) (size 0.8) (drill 0.4) (layers "F.Cu" "B.Cu") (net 14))
 (via (at 196.2 118.15) (size 0.8) (drill 0.4) (layers "F.Cu" "B.Cu") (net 14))
 (segment (start 182.65 118.05) (end 184.9 118.05) (width 0.25) (layer "B.Cu") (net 14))
 (segment (start 196.25 118.05) (end 196.35 117.95) (width 0.25) (layer "B.Cu") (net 14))
 (segment (start 184.9 118.05) (end 196.2 118.15) (width 0.25) (layer "B.Cu") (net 14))
 (segment (start 182.65 128.99) (end 182.65 118.05) (width 0.25) (layer "B.Cu") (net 14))
 (segment (start 179.45 132.19) (end 182.65 128.99) (width 0.25) (layer "B.Cu") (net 14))
 (segment (start 196.2 118.15) (end 196.25 118.05) (width 0.25) (layer "B.Cu") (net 14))
 (segment (start 184.8459 124.5) (end 182.06 124.5) (width 0.25) (layer "F.Cu") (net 13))
 (segment (start 182.06 124.5) (end 179.45 127.11) (width 0.25) (layer "F.Cu") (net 13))
 (segment (start 180.626001 123.206001) (end 179.45 122.03) (width 0.25) (layer "F.Cu") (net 11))
 (segment (start 186.1234 123.9734) (end 185.356001 123.206001) (width 0.25) (layer "F.Cu") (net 11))
 (segment (start 184.8459 128.499999) (end 186.1234 127.222499) (width 0.25) (layer "F.Cu") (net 11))
 (segment (start 185.356001 123.206001) (end 180.626001 123.206001) (width 0.25) (layer "F.Cu") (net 11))
 (segment (start 186.1234 127.222499) (end 186.1234 123.9734) (width 0.25) (layer "F.Cu") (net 11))
 (segment (start 178.963299 128.285) (end 178.25 127.571701) (width 0.25) (layer "F.Cu") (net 12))
 (segment (start 184.8459 126.500001) (end 183.060901 128.285) (width 0.25) (layer "F.Cu") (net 12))
 (segment (start 178.25 125.77) (end 179.45 124.57) (width 0.25) (layer "F.Cu") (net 12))
 (segment (start 183.060901 128.285) (end 178.963299 128.285) (width 0.25) (layer "F.Cu") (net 12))
 (segment (start 178.25 127.571701) (end 178.25 125.77) (width 0.25) (layer "F.Cu") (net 12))
 (segment (start 187.3 116.95) (end 188.35 118) (width 0.25) (layer "F.Cu") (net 9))
 (segment (start 184.8459 130.500001) (end 188.35 126.995901) (width 0.25) (layer "F.Cu") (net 9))
 (segment (start 188.35 126.995901) (end 188.35 118) (width 0.25) (layer "F.Cu") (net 9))
 (segment (start 179.45 116.95) (end 187.3 116.95) (width 0.25) (layer "F.Cu") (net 9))
 (segment (start 184.8459 134.5) (end 182.6 134.5) (width 0.25) (layer "F.Cu") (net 1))
 (segment (start 182.6 134.5) (end 182.4 134.3) (width 0.25) (layer "F.Cu") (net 1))
 (via (at 182.4 134.3) (size 0.8) (drill 0.4) (layers "F.Cu" "B.Cu") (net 1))
 (segment (start 204.9 116.91) (end 199.74 116.91) (width 0.25) (layer "B.Cu") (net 1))
 (segment (start 199.74 116.91) (end 182.4 134.25) (width 0.25) (layer "B.Cu") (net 1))
 (segment (start 182.4 134.25) (end 182.4 134.3) (width 0.25) (layer "B.Cu") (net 1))
 (segment (start 182.4 134.3) (end 182.35 134.3) (width 0.25) (layer "B.Cu") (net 1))
 (segment (start 182.35 134.3) (end 182.35 134.3) (width 0.25) (layer "B.Cu") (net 1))
 (segment (start 199.5525 132.499999) (end 203.671702 132.499999) (width 0.25) (layer "F.Cu") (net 3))
 (segment (start 206.075 130.096701) (end 206.075 123.165) (width 0.25) (layer "F.Cu") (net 3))
 (segment (start 203.671702 132.499999) (end 206.075 130.096701) (width 0.25) (layer "F.Cu") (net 3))
 (segment (start 206.075 123.165) (end 204.9 121.99) (width 0.25) (layer "F.Cu") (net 3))
 (segment (start 199.5525 124.5) (end 202.33 124.5) (width 0.25) (layer "F.Cu") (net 5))
 (segment (start 202.33 124.5) (end 204.9 127.07) (width 0.25) (layer "F.Cu") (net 5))
 (segment (start 201.399999 130.500001) (end 202.2 129.75) (width 0.25) (layer "F.Cu") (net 2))
 (segment (start 202.2 129.75) (end 202.025 129.875) (width 0.25) (layer "F.Cu") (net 2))
 (segment (start 199.5525 130.500001) (end 201.399999 130.500001) (width 0.25) (layer "F.Cu") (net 2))
 (via (at 202.2 129.75) (size 0.8) (drill 0.4) (layers "F.Cu" "B.Cu") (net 2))
 (segment (start 204.9 119.45) (end 202.2 122.15) (width 0.25) (layer "B.Cu") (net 2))
 (segment (start 202.2 122.15) (end 202.2 129.75) (width 0.25) (layer "B.Cu") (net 2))
 (segment (start 202.716001 131.793999) (end 204.9 129.61) (width 0.25) (layer "F.Cu") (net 6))
 (segment (start 208.25 128.45) (end 208.25 128.5) (width 0.25) (layer "F.Cu") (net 6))
 (segment (start 199.1588 117.75) (end 201.1738 115.735) (width 0.25) (layer "F.Cu") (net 6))
 (segment (start 208.25 128.35) (end 208.3 128.4) (width 0.25) (layer "F.Cu") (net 6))
 (segment (start 185.5519 131.793999) (end 202.716001 131.793999) (width 0.25) (layer "F.Cu") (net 6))
 (segment (start 201.1738 115.735) (end 206.985 115.735) (width 0.25) (layer "F.Cu") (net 6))
 (segment (start 208.25 117) (end 208.25 128.35) (width 0.25) (layer "F.Cu") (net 6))
 (segment (start 208.3 128.4) (end 208.25 128.45) (width 0.25) (layer "F.Cu") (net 6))
 (segment (start 206.985 115.735) (end 208.25 117) (width 0.25) (layer "F.Cu") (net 6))
 (segment (start 184.8459 132.499999) (end 185.5519 131.793999) (width 0.25) (layer "F.Cu") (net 6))
 (via (at 208.3 128.4) (size 0.8) (drill 0.4) (layers "F.Cu" "B.Cu") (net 6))
 (segment (start 204.9 129.61) (end 207.09 129.61) (width 0.25) (layer "B.Cu") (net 6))
 (segment (start 207.09 129.61) (end 208.3 128.4) (width 0.25) (layer "B.Cu") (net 6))
 (segment (start 199.5525 122.499999) (end 202.869999 122.499999) (width 0.25) (layer "F.Cu") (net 4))
 (segment (start 202.869999 122.499999) (end 204.9 124.53) (width 0.25) (layer "F.Cu") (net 4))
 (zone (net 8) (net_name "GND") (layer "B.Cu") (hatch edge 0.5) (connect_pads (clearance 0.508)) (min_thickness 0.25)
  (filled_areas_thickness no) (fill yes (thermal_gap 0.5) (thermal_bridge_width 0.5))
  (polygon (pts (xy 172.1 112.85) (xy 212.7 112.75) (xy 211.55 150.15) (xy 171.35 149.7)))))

